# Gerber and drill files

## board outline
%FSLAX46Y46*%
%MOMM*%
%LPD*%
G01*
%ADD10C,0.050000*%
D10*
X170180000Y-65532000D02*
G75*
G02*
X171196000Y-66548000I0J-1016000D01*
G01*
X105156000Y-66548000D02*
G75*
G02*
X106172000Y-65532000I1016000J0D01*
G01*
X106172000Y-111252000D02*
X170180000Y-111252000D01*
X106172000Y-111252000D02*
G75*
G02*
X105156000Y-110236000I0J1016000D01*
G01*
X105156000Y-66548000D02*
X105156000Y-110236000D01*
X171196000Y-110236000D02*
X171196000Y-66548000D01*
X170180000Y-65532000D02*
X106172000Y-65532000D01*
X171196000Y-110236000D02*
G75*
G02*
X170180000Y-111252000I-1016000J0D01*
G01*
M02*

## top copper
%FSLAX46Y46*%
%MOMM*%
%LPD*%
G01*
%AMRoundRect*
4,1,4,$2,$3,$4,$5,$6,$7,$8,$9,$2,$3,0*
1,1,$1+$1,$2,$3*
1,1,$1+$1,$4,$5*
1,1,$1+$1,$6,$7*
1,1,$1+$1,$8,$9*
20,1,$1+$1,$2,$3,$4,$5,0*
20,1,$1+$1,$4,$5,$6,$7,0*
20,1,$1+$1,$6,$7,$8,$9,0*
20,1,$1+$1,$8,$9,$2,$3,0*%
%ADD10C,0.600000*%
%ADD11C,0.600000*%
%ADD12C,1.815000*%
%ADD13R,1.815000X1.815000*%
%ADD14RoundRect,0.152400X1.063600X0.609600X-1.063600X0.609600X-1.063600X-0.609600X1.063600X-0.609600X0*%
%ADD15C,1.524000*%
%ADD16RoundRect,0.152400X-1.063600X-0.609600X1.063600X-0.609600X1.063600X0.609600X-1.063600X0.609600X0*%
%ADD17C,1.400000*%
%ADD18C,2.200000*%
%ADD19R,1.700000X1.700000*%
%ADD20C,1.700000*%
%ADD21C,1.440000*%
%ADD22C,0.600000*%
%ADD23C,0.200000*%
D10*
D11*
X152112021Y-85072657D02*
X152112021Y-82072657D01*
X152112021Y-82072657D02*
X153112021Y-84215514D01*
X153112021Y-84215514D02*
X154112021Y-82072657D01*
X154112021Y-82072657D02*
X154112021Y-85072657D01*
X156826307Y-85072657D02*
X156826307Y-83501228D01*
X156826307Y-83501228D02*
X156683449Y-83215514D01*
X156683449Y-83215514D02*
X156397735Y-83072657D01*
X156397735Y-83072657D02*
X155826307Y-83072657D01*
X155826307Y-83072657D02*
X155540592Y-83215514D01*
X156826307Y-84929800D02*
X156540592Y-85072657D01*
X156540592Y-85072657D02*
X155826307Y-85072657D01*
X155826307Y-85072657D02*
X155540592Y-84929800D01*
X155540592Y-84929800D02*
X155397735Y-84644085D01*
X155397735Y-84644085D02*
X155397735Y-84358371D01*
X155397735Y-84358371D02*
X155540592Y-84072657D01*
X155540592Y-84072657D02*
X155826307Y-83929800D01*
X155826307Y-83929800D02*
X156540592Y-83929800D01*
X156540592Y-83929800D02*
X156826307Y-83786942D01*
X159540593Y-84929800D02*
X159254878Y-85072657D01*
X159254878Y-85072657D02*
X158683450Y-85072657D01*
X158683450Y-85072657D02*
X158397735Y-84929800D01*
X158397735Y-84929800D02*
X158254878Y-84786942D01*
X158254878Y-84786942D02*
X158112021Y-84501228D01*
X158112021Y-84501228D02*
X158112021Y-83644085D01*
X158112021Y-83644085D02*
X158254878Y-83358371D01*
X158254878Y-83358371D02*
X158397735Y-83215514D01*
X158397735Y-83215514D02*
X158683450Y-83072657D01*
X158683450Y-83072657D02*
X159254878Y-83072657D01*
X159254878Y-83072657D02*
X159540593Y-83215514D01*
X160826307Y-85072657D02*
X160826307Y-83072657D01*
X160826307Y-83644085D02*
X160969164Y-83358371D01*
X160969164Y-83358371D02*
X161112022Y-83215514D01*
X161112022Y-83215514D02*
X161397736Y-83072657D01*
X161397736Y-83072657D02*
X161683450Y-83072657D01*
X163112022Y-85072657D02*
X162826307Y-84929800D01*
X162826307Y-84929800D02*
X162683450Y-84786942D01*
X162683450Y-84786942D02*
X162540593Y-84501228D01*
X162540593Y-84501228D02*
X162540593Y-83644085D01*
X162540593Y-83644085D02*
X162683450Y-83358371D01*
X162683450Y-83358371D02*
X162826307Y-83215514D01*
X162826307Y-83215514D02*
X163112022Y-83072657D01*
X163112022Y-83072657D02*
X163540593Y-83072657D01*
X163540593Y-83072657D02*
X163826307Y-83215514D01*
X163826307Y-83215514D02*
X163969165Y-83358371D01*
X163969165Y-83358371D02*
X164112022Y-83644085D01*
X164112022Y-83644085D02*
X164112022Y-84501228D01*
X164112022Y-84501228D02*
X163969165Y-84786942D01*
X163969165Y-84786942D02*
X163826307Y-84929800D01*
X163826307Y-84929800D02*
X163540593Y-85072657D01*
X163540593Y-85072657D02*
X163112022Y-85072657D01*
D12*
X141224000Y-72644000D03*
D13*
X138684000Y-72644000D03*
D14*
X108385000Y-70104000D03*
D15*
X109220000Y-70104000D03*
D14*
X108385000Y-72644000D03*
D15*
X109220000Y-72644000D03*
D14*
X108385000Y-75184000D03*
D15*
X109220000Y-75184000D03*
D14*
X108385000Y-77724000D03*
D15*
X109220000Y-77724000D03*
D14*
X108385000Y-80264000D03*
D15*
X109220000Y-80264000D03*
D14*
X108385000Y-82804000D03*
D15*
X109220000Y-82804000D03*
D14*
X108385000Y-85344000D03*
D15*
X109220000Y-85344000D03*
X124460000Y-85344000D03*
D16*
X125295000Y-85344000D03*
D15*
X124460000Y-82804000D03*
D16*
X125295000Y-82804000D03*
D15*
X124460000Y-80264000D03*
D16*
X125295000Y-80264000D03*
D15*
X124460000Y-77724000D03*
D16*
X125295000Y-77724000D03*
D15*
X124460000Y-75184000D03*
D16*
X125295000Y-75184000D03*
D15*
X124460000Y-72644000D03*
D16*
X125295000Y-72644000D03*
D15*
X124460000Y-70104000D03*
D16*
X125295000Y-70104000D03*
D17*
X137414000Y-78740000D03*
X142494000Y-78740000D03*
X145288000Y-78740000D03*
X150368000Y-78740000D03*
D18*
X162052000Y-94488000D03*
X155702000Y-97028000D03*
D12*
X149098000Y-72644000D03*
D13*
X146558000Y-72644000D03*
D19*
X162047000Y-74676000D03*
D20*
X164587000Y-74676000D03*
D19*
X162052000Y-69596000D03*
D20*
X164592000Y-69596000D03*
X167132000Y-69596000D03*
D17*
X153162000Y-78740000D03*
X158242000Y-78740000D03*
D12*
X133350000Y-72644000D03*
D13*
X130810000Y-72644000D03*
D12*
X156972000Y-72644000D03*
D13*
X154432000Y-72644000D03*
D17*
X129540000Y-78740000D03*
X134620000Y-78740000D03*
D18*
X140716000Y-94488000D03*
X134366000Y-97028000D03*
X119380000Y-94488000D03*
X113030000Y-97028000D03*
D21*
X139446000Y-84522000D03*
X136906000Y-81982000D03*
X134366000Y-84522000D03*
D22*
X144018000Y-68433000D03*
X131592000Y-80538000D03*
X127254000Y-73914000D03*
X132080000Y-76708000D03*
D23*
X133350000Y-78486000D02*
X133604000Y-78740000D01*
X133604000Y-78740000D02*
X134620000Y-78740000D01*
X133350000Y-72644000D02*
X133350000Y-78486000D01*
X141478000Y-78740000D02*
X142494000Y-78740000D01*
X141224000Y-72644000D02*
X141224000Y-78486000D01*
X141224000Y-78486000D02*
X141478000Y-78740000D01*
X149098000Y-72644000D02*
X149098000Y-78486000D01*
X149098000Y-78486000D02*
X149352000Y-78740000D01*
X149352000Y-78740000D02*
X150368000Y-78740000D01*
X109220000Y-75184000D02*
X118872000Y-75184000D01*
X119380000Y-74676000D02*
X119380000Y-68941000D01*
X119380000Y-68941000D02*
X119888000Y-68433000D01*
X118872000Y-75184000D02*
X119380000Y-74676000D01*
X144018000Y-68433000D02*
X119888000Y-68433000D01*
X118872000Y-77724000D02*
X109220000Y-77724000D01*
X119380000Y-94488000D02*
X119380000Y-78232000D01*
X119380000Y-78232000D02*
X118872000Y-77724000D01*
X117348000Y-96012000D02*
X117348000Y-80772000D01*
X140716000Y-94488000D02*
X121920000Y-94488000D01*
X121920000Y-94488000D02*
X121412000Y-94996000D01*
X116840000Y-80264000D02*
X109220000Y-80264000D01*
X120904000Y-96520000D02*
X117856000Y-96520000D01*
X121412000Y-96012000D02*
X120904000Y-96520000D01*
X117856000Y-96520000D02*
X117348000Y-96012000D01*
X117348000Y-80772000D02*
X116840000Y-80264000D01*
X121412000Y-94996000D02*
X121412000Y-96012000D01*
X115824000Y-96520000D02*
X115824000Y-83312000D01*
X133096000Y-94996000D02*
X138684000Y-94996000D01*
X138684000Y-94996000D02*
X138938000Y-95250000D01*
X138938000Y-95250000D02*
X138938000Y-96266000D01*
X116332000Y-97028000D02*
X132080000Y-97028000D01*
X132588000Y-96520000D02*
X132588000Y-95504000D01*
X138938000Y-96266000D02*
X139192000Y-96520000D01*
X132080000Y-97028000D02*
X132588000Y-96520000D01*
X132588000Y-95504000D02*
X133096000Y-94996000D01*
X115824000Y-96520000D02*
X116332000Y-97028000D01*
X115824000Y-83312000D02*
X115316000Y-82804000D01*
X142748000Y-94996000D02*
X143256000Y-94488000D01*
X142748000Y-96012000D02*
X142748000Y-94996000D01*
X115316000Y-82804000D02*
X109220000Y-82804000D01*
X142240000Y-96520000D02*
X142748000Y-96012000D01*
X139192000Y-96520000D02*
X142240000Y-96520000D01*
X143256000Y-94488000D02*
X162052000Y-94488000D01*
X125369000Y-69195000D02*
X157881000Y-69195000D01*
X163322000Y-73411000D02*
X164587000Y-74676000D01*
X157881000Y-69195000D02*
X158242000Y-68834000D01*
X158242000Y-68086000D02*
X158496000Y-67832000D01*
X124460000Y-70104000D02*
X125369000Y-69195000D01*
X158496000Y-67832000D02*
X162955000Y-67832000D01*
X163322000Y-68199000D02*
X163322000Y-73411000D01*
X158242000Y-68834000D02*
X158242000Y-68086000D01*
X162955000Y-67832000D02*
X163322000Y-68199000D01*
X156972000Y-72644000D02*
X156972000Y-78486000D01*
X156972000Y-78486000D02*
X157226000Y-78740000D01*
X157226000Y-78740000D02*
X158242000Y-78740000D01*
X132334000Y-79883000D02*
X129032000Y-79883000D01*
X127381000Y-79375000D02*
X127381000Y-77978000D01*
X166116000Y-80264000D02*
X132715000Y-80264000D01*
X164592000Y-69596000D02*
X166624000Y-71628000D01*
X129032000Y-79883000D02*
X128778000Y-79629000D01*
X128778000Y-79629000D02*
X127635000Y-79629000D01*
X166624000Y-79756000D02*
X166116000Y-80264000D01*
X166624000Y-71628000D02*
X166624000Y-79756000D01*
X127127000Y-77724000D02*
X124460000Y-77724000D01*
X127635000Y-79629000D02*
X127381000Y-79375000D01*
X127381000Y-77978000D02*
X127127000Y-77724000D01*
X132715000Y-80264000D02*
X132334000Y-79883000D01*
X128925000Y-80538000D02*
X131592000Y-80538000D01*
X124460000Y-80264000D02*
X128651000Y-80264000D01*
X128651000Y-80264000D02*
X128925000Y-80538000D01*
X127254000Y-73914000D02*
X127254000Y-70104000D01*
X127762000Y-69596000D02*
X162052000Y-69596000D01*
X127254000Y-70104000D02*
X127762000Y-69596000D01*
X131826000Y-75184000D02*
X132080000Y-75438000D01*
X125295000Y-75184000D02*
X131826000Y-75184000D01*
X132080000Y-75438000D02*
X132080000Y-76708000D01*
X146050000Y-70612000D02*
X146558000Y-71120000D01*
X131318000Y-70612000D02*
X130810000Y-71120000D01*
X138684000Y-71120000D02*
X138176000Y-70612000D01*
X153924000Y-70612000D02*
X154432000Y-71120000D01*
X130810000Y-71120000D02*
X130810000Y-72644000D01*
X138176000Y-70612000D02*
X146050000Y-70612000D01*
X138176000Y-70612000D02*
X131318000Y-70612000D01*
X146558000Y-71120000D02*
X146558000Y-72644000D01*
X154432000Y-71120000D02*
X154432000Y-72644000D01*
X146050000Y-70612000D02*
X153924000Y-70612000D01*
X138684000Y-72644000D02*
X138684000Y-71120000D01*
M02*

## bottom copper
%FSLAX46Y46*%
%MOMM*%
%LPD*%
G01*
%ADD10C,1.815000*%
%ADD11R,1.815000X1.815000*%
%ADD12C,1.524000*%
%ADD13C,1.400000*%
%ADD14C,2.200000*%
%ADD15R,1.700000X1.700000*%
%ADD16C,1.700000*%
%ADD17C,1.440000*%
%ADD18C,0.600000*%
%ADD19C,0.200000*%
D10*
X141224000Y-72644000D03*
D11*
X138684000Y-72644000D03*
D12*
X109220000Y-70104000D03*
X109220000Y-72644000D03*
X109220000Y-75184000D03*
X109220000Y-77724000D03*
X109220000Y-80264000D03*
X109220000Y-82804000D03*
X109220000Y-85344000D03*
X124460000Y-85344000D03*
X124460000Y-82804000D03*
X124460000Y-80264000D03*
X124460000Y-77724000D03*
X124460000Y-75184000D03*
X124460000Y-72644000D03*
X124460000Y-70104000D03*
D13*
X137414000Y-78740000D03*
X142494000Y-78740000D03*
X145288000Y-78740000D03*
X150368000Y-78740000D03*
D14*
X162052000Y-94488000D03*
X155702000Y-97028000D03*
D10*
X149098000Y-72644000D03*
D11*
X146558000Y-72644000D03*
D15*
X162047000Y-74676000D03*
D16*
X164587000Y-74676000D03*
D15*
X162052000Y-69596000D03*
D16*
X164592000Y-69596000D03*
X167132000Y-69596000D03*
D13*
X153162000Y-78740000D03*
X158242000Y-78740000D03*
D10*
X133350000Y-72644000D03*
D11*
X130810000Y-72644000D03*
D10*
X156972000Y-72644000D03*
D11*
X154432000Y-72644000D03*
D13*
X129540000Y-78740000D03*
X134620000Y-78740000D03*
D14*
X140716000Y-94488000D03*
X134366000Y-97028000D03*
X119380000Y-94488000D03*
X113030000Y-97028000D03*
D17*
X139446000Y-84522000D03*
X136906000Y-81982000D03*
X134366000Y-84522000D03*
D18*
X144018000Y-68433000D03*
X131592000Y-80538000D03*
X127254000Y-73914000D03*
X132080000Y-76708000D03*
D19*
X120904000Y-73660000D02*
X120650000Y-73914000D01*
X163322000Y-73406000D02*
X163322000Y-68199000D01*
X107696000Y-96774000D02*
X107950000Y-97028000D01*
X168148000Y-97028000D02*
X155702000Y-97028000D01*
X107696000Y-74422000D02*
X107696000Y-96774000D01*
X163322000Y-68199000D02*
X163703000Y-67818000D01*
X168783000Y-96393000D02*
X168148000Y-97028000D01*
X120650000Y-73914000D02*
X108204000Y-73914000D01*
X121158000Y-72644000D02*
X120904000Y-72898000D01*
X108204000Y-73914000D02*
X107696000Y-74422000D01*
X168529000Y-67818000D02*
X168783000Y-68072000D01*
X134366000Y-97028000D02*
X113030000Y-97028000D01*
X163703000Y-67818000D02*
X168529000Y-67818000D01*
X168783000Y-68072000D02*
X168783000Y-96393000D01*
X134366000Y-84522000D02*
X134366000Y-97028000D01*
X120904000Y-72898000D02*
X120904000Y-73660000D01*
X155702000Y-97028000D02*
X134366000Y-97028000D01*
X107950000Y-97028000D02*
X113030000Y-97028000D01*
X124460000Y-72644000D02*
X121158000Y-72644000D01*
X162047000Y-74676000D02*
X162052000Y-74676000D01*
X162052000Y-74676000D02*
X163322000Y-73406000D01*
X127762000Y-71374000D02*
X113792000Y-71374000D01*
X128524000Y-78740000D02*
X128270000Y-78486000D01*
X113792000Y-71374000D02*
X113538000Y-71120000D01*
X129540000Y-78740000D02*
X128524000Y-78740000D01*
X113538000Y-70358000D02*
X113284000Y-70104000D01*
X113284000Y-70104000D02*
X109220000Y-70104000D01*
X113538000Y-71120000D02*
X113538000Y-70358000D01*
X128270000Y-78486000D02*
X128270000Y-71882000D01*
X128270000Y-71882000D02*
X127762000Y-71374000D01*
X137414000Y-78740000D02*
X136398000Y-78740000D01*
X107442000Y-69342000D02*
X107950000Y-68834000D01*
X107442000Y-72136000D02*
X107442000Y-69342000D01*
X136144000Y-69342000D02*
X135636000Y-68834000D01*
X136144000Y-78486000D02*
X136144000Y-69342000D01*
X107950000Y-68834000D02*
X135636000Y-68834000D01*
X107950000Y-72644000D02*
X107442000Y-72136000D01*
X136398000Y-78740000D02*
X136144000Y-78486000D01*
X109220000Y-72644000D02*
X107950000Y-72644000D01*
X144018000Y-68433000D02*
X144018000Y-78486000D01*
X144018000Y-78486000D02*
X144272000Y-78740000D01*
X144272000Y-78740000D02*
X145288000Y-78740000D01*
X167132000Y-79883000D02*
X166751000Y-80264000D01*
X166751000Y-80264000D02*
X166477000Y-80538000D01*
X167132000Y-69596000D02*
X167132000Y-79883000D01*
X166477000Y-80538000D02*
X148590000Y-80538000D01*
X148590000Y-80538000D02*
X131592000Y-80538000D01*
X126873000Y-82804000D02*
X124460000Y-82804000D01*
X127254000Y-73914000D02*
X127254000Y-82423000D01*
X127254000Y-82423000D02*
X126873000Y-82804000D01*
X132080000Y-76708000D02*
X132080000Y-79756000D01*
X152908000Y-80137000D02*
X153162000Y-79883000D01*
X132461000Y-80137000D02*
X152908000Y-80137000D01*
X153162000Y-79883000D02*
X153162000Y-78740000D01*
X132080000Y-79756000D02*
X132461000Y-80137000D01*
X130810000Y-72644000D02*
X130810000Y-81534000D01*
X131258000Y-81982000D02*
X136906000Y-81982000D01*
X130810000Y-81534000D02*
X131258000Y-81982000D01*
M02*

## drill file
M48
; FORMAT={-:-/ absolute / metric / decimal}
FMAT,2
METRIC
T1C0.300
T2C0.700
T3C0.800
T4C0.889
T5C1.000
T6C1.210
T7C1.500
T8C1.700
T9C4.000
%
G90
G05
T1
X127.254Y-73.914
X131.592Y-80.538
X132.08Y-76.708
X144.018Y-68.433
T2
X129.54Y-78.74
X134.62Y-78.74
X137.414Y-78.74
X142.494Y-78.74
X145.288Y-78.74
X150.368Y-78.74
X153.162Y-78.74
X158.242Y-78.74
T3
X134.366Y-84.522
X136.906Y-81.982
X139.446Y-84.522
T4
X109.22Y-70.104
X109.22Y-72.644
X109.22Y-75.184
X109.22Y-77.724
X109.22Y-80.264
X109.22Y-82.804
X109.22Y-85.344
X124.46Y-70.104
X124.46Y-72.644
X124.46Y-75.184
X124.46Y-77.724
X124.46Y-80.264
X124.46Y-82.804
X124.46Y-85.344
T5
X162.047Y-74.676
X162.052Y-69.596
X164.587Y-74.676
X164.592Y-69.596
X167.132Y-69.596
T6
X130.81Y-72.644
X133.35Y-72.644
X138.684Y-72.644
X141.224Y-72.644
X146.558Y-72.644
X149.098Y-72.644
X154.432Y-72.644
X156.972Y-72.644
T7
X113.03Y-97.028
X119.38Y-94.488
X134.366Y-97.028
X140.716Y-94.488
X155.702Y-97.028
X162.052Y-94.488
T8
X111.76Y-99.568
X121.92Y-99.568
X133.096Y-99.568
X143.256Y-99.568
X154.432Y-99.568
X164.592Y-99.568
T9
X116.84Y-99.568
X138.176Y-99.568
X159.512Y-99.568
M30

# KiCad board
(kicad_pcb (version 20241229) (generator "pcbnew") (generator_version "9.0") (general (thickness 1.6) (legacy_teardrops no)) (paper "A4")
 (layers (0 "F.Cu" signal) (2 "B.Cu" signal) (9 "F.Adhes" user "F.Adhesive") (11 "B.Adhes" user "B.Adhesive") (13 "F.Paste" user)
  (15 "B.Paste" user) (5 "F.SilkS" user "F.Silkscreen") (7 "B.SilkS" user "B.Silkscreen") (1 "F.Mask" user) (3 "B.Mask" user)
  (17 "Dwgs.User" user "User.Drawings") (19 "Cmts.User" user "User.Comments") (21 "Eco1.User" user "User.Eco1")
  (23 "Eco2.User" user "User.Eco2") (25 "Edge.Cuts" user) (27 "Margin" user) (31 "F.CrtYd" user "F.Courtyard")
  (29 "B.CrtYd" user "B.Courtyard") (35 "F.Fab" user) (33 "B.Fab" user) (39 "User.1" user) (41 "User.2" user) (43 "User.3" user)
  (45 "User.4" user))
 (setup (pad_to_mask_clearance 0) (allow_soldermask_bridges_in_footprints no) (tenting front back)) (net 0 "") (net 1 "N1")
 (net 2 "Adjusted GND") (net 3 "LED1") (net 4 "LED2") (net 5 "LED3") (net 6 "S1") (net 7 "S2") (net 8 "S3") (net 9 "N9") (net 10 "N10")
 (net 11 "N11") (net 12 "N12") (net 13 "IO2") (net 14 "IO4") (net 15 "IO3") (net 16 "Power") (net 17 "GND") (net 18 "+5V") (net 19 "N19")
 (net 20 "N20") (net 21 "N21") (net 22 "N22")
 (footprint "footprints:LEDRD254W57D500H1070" (layer "F.Cu") (at 139.954 72.644)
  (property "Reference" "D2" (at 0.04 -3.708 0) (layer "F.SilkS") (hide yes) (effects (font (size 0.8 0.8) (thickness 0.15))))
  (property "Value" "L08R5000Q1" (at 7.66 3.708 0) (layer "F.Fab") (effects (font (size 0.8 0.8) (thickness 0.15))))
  (pad "A" thru_hole circle (at 1.27 0) (size 1.815 1.815) (drill 1.21) (layers "*.Cu" "*.Mask") (remove_unused_layers no) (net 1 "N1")
   (solder_mask_margin 0.102))
  (pad "C" thru_hole rect (at -1.27 0) (size 1.815 1.815) (drill 1.21) (layers "*.Cu" "*.Mask") (remove_unused_layers no)
   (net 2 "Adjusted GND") (solder_mask_margin 0.102)))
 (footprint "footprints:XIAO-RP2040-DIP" (layer "F.Cu") (at 116.84 77.724)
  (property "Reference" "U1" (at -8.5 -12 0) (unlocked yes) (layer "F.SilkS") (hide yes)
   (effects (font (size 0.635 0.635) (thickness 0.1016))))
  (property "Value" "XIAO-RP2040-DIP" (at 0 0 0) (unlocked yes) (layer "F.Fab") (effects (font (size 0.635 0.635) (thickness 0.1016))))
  (pad "1" smd roundrect (at -8.455 -7.62 180) (size 2.432 1.524) (layers "F.Cu" "F.Mask") (roundrect_rratio 0.1) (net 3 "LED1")
   (thermal_bridge_angle 45))
  (pad "1" thru_hole circle (at -7.62 -7.62 180) (size 1.524 1.524) (drill 0.889) (layers "*.Cu" "*.Mask") (remove_unused_layers no)
   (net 3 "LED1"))
  (pad "2" smd roundrect (at -8.455 -5.08 180) (size 2.432 1.524) (layers "F.Cu" "F.Mask") (roundrect_rratio 0.1) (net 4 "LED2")
   (thermal_bridge_angle 45))
  (pad "2" thru_hole circle (at -7.62 -5.08 180) (size 1.524 1.524) (drill 0.889) (layers "*.Cu" "*.Mask") (remove_unused_layers no)
   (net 4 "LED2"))
  (pad "3" smd roundrect (at -8.455 -2.54 180) (size 2.432 1.524) (layers "F.Cu" "F.Mask") (roundrect_rratio 0.1) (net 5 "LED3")
   (thermal_bridge_angle 45))
  (pad "3" thru_hole circle (at -7.62 -2.54 180) (size 1.524 1.524) (drill 0.889) (layers "*.Cu" "*.Mask") (remove_unused_layers no)
   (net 5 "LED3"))
  (pad "4" smd roundrect (at -8.455 0 180) (size 2.432 1.524) (layers "F.Cu" "F.Mask") (roundrect_rratio 0.1) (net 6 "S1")
   (thermal_bridge_angle 45))
  (pad "4" thru_hole circle (at -7.62 0 180) (size 1.524 1.524) (drill 0.889) (layers "*.Cu" "*.Mask") (remove_unused_layers no)
   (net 6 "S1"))
  (pad "5" smd roundrect (at -8.455 2.54 180) (size 2.432 1.524) (layers "F.Cu" "F.Mask") (roundrect_rratio 0.1) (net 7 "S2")
   (thermal_bridge_angle 45))
  (pad "5" thru_hole circle (at -7.62 2.54 180) (size 1.524 1.524) (drill 0.889) (layers "*.Cu" "*.Mask") (remove_unused_layers no)
   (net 7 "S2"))
  (pad "6" smd roundrect (at -8.455 5.08 180) (size 2.432 1.524) (layers "F.Cu" "F.Mask") (roundrect_rratio 0.1) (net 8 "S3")
   (thermal_bridge_angle 45))
  (pad "6" thru_hole circle (at -7.62 5.08 180) (size 1.524 1.524) (drill 0.889) (layers "*.Cu" "*.Mask") (remove_unused_layers no)
   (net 8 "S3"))
  (pad "7" smd roundrect (at -8.455 7.62 180) (size 2.432 1.524) (layers "F.Cu" "F.Mask") (roundrect_rratio 0.1) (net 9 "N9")
   (thermal_bridge_angle 45))
  (pad "7" thru_hole circle (at -7.62 7.62 180) (size 1.524 1.524) (drill 0.889) (layers "*.Cu" "*.Mask") (remove_unused_layers no)
   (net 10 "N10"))
  (pad "8" thru_hole circle (at 7.62 7.62) (size 1.524 1.524) (drill 0.889) (layers "*.Cu" "*.Mask") (remove_unused_layers no)
   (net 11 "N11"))
  (pad "8" smd roundrect (at 8.455 7.62) (size 2.432 1.524) (layers "F.Cu" "F.Mask") (roundrect_rratio 0.1) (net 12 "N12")
   (thermal_bridge_angle 45))
  (pad "9" thru_hole circle (at 7.62 5.08) (size 1.524 1.524) (drill 0.889) (layers "*.Cu" "*.Mask") (remove_unused_layers no)
   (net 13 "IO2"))
  (pad "9" smd roundrect (at 8.455 5.08) (size 2.432 1.524) (layers "F.Cu" "F.Mask") (roundrect_rratio 0.1) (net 13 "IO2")
   (thermal_bridge_angle 45))
  (pad "10" thru_hole circle (at 7.62 2.54) (size 1.524 1.524) (drill 0.889) (layers "*.Cu" "*.Mask") (remove_unused_layers no)
   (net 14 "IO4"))
  (pad "10" smd roundrect (at 8.455 2.54) (size 2.432 1.524) (layers "F.Cu" "F.Mask") (roundrect_rratio 0.1) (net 14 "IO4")
   (thermal_bridge_angle 45))
  (pad "11" thru_hole circle (at 7.62 0) (size 1.524 1.524) (drill 0.889) (layers "*.Cu" "*.Mask") (remove_unused_layers no) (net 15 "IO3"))
  (pad "11" smd roundrect (at 8.455 0) (size 2.432 1.524) (layers "F.Cu" "F.Mask") (roundrect_rratio 0.1) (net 15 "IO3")
   (thermal_bridge_angle 45))
  (pad "12" thru_hole circle (at 7.62 -2.54) (size 1.524 1.524) (drill 0.889) (layers "*.Cu" "*.Mask") (remove_unused_layers no)
   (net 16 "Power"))
  (pad "12" smd roundrect (at 8.455 -2.54) (size 2.432 1.524) (layers "F.Cu" "F.Mask") (roundrect_rratio 0.1) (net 16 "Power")
   (thermal_bridge_angle 45))
  (pad "13" thru_hole circle (at 7.62 -5.08) (size 1.524 1.524) (drill 0.889) (layers "*.Cu" "*.Mask") (remove_unused_layers no)
   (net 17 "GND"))
  (pad "13" smd roundrect (at 8.455 -5.08) (size 2.432 1.524) (layers "F.Cu" "F.Mask") (roundrect_rratio 0.1) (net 17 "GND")
   (thermal_bridge_angle 45))
  (pad "14" thru_hole circle (at 7.62 -7.62) (size 1.524 1.524) (drill 0.889) (layers "*.Cu" "*.Mask") (remove_unused_layers no)
   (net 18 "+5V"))
  (pad "14" smd roundrect (at 8.455 -7.62) (size 2.432 1.524) (layers "F.Cu" "F.Mask") (roundrect_rratio 0.1) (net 18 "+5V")
   (thermal_bridge_angle 45)))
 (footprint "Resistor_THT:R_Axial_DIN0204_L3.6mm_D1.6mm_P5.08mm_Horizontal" (layer "F.Cu") (at 137.414 78.74)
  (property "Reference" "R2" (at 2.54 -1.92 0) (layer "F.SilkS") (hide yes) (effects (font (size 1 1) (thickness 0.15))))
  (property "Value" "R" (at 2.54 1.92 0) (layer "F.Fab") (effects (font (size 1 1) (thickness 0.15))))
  (pad "1" thru_hole circle (at 0 0) (size 1.4 1.4) (drill 0.7) (layers "*.Cu" "*.Mask") (remove_unused_layers no) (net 4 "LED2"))
  (pad "2" thru_hole circle (at 5.08 0) (size 1.4 1.4) (drill 0.7) (layers "*.Cu" "*.Mask") (remove_unused_layers no) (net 1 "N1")))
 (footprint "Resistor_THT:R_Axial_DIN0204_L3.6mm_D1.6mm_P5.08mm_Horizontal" (layer "F.Cu") (at 145.288 78.74)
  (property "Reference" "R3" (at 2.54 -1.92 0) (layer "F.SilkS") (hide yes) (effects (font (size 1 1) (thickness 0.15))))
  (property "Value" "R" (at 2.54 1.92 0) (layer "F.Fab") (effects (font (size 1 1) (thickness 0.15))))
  (pad "1" thru_hole circle (at 0 0) (size 1.4 1.4) (drill 0.7) (layers "*.Cu" "*.Mask") (remove_unused_layers no) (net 5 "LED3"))
  (pad "2" thru_hole circle (at 5.08 0) (size 1.4 1.4) (drill 0.7) (layers "*.Cu" "*.Mask") (remove_unused_layers no) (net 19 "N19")))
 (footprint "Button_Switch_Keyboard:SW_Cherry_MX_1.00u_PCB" (layer "F.Cu") (at 162.052 94.488)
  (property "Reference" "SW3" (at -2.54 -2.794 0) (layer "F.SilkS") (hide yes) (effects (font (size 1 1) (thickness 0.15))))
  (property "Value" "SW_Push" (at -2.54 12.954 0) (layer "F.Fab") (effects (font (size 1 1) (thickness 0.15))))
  (pad "" np_thru_hole circle (at -7.62 5.08) (size 1.7 1.7) (drill 1.7) (layers "*.Cu" "*.Mask"))
  (pad "" np_thru_hole circle (at -2.54 5.08) (size 4 4) (drill 4) (layers "*.Cu" "*.Mask"))
  (pad "" np_thru_hole circle (at 2.54 5.08) (size 1.7 1.7) (drill 1.7) (layers "*.Cu" "*.Mask"))
  (pad "1" thru_hole circle (at 0 0) (size 2.2 2.2) (drill 1.5) (layers "*.Cu" "*.Mask") (remove_unused_layers no) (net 8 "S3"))
  (pad "2" thru_hole circle (at -6.35 2.54) (size 2.2 2.2) (drill 1.5) (layers "*.Cu" "*.Mask") (remove_unused_layers no) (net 17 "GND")))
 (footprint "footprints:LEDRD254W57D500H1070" (layer "F.Cu") (at 147.828 72.644)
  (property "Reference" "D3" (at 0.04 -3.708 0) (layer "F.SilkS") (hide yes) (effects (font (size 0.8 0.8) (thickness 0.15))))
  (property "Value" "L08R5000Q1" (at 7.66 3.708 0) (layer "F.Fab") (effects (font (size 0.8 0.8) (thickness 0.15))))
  (pad "A" thru_hole circle (at 1.27 0) (size 1.815 1.815) (drill 1.21) (layers "*.Cu" "*.Mask") (remove_unused_layers no) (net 19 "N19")
   (solder_mask_margin 0.102))
  (pad "C" thru_hole rect (at -1.27 0) (size 1.815 1.815) (drill 1.21) (layers "*.Cu" "*.Mask") (remove_unused_layers no)
   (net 2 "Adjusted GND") (solder_mask_margin 0.102)))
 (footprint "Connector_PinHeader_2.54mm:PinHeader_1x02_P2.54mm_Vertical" (layer "F.Cu") (at 162.047 74.676 90)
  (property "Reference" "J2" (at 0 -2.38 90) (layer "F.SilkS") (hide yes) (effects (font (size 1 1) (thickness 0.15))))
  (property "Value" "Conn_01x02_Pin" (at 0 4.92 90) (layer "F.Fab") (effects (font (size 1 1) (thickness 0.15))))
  (pad "1" thru_hole rect (at 0 0 90) (size 1.7 1.7) (drill 1) (layers "*.Cu" "*.Mask") (remove_unused_layers no) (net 17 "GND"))
  (pad "2" thru_hole circle (at 0 2.54 90) (size 1.7 1.7) (drill 1) (layers "*.Cu" "*.Mask") (remove_unused_layers no) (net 18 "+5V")))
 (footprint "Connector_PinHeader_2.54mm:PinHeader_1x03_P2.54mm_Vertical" (layer "F.Cu") (at 162.052 69.596 90)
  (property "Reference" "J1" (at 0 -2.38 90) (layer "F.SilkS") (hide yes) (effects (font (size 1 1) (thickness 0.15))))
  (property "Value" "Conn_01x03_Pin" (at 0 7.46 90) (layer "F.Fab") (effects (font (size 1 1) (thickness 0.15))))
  (pad "1" thru_hole rect (at 0 0 90) (size 1.7 1.7) (drill 1) (layers "*.Cu" "*.Mask") (remove_unused_layers no) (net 13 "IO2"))
  (pad "2" thru_hole circle (at 0 2.54 90) (size 1.7 1.7) (drill 1) (layers "*.Cu" "*.Mask") (remove_unused_layers no) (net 15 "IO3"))
  (pad "3" thru_hole circle (at 0 5.08 90) (size 1.7 1.7) (drill 1) (layers "*.Cu" "*.Mask") (remove_unused_layers no) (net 14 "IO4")))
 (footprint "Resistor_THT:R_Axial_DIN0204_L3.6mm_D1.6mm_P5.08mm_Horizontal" (layer "F.Cu") (at 153.162 78.74)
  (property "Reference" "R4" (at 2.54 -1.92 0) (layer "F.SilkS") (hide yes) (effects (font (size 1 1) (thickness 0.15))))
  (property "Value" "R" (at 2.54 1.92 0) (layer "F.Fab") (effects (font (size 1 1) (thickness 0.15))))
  (pad "1" thru_hole circle (at 0 0) (size 1.4 1.4) (drill 0.7) (layers "*.Cu" "*.Mask") (remove_unused_layers no) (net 16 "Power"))
  (pad "2" thru_hole circle (at 5.08 0) (size 1.4 1.4) (drill 0.7) (layers "*.Cu" "*.Mask") (remove_unused_layers no) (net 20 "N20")))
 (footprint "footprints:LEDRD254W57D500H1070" (layer "F.Cu") (at 132.08 72.644)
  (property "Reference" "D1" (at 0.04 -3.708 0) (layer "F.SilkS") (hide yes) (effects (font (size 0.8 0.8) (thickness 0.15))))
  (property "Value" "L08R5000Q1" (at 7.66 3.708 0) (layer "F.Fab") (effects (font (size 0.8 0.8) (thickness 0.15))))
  (pad "A" thru_hole circle (at 1.27 0) (size 1.815 1.815) (drill 1.21) (layers "*.Cu" "*.Mask") (remove_unused_layers no) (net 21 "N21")
   (solder_mask_margin 0.102))
  (pad "C" thru_hole rect (at -1.27 0) (size 1.815 1.815) (drill 1.21) (layers "*.Cu" "*.Mask") (remove_unused_layers no)
   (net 2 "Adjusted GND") (solder_mask_margin 0.102)))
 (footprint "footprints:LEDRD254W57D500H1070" (layer "F.Cu") (at 155.702 72.644)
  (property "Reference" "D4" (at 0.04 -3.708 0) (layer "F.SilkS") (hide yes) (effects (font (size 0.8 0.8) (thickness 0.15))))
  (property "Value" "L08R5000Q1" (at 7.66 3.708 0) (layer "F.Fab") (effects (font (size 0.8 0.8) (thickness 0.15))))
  (pad "A" thru_hole circle (at 1.27 0) (size 1.815 1.815) (drill 1.21) (layers "*.Cu" "*.Mask") (remove_unused_layers no) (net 20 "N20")
   (solder_mask_margin 0.102))
  (pad "C" thru_hole rect (at -1.27 0) (size 1.815 1.815) (drill 1.21) (layers "*.Cu" "*.Mask") (remove_unused_layers no)
   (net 2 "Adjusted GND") (solder_mask_margin 0.102)))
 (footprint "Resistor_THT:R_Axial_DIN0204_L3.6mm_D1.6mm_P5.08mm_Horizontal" (layer "F.Cu") (at 129.54 78.74)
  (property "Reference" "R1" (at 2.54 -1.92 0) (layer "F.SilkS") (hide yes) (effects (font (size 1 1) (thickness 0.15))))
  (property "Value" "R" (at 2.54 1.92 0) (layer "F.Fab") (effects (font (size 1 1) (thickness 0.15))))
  (pad "1" thru_hole circle (at 0 0) (size 1.4 1.4) (drill 0.7) (layers "*.Cu" "*.Mask") (remove_unused_layers no) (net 3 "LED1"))
  (pad "2" thru_hole circle (at 5.08 0) (size 1.4 1.4) (drill 0.7) (layers "*.Cu" "*.Mask") (remove_unused_layers no) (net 21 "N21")))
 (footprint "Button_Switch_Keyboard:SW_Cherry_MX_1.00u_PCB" (layer "F.Cu") (at 140.716 94.488)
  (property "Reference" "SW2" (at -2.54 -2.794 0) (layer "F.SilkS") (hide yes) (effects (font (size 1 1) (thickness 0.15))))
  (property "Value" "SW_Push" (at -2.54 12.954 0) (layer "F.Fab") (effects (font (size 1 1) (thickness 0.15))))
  (pad "" np_thru_hole circle (at -7.62 5.08) (size 1.7 1.7) (drill 1.7) (layers "*.Cu" "*.Mask"))
  (pad "" np_thru_hole circle (at -2.54 5.08) (size 4 4) (drill 4) (layers "*.Cu" "*.Mask"))
  (pad "" np_thru_hole circle (at 2.54 5.08) (size 1.7 1.7) (drill 1.7) (layers "*.Cu" "*.Mask"))
  (pad "1" thru_hole circle (at 0 0) (size 2.2 2.2) (drill 1.5) (layers "*.Cu" "*.Mask") (remove_unused_layers no) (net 7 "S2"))
  (pad "2" thru_hole circle (at -6.35 2.54) (size 2.2 2.2) (drill 1.5) (layers "*.Cu" "*.Mask") (remove_unused_layers no) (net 17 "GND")))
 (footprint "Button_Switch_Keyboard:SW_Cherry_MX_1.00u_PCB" (layer "F.Cu") (at 119.38 94.488)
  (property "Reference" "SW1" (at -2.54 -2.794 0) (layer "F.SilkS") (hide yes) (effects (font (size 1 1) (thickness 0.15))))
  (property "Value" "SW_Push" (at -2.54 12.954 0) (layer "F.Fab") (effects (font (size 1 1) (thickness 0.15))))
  (pad "" np_thru_hole circle (at -7.62 5.08) (size 1.7 1.7) (drill 1.7) (layers "*.Cu" "*.Mask"))
  (pad "" np_thru_hole circle (at -2.54 5.08) (size 4 4) (drill 4) (layers "*.Cu" "*.Mask"))
  (pad "" np_thru_hole circle (at 2.54 5.08) (size 1.7 1.7) (drill 1.7) (layers "*.Cu" "*.Mask"))
  (pad "1" thru_hole circle (at 0 0) (size 2.2 2.2) (drill 1.5) (layers "*.Cu" "*.Mask") (remove_unused_layers no) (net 6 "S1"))
  (pad "2" thru_hole circle (at -6.35 2.54) (size 2.2 2.2) (drill 1.5) (layers "*.Cu" "*.Mask") (remove_unused_layers no) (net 17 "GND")))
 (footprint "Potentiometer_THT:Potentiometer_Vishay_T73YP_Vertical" (layer "F.Cu") (at 139.446 84.522 90)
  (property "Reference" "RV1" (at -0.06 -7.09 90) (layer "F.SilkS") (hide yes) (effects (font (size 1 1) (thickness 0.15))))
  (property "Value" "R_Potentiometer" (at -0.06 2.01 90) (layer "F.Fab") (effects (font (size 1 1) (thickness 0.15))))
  (pad "1" thru_hole circle (at 0 0 90) (size 1.44 1.44) (drill 0.8) (layers "*.Cu" "*.Mask") (remove_unused_layers no) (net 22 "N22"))
  (pad "2" thru_hole circle (at 2.54 -2.54 90) (size 1.44 1.44) (drill 0.8) (layers "*.Cu" "*.Mask") (remove_unused_layers no)
   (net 2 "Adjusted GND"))
  (pad "3" thru_hole circle (at 0 -5.08 90) (size 1.44 1.44) (drill 0.8) (layers "*.Cu" "*.Mask") (remove_unused_layers no) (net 17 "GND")))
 (gr_arc (start 170.18 65.532) (mid 170.89842 65.82958) (end 171.196 66.548) (stroke (width 0.05) (type default)) (layer "Edge.Cuts"))
 (gr_arc (start 105.156 66.548) (mid 105.45358 65.82958) (end 106.172 65.532) (stroke (width 0.05) (type default)) (layer "Edge.Cuts"))
 (gr_line (start 106.172 111.252) (end 170.18 111.252) (stroke (width 0.05) (type default)) (layer "Edge.Cuts"))
 (gr_arc (start 106.172 111.252) (mid 105.45358 110.95442) (end 105.156 110.236) (stroke (width 0.05) (type default)) (layer "Edge.Cuts"))
 (gr_line (start 105.156 66.548) (end 105.156 110.236) (stroke (width 0.05) (type default)) (layer "Edge.Cuts"))
 (gr_line (start 171.196 110.236) (end 171.196 66.548) (stroke (width 0.05) (type default)) (layer "Edge.Cuts"))
 (gr_line (start 170.18 65.532) (end 106.172 65.532) (stroke (width 0.05) (type default)) (layer "Edge.Cuts"))
 (gr_arc (start 171.196 110.236) (mid 170.89842 110.95442) (end 170.18 111.252) (stroke (width 0.05) (type default)) (layer "Edge.Cuts"))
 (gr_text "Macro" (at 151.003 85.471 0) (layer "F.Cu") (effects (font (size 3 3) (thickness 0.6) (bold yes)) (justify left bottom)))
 (segment (start 120.904 73.66) (end 120.65 73.914) (width 0.2) (layer "B.Cu") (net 17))
 (segment (start 163.322 73.406) (end 163.322 68.199) (width 0.2) (layer "B.Cu") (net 17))
 (segment (start 107.696 96.774) (end 107.95 97.028) (width 0.2) (layer "B.Cu") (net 17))
 (segment (start 168.148 97.028) (end 155.702 97.028) (width 0.2) (layer "B.Cu") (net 17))
 (segment (start 107.696 74.422) (end 107.696 96.774) (width 0.2) (layer "B.Cu") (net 17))
 (segment (start 163.322 68.199) (end 163.703 67.818) (width 0.2) (layer "B.Cu") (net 17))
 (segment (start 168.783 96.393) (end 168.148 97.028) (width 0.2) (layer "B.Cu") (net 17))
 (segment (start 120.65 73.914) (end 108.204 73.914) (width 0.2) (layer "B.Cu") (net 17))
 (segment (start 121.158 72.644) (end 120.904 72.898) (width 0.2) (layer "B.Cu") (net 17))
 (segment (start 108.204 73.914) (end 107.696 74.422) (width 0.2) (layer "B.Cu") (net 17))
 (segment (start 168.529 67.818) (end 168.783 68.072) (width 0.2) (layer "B.Cu") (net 17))
 (segment (start 134.366 97.028) (end 113.03 97.028) (width 0.2) (layer "B.Cu") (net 17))
 (segment (start 163.703 67.818) (end 168.529 67.818) (width 0.2) (layer "B.Cu") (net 17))
 (segment (start 168.783 68.072) (end 168.783 96.393) (width 0.2) (layer "B.Cu") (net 17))
 (segment (start 134.366 84.522) (end 134.366 97.028) (width 0.2) (layer "B.Cu") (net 17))
 (segment (start 120.904 72.898) (end 120.904 73.66) (width 0.2) (layer "B.Cu") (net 17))
 (segment (start 155.702 97.028) (end 134.366 97.028) (width 0.2) (layer "B.Cu") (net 17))
 (segment (start 107.95 97.028) (end 113.03 97.028) (width 0.2) (layer "B.Cu") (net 17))
 (segment (start 124.46 72.644) (end 121.158 72.644) (width 0.2) (layer "B.Cu") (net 17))
 (segment (start 162.047 74.676) (end 162.052 74.676) (width 0.2) (layer "B.Cu") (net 17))
 (segment (start 162.052 74.676) (end 163.322 73.406) (width 0.2) (layer "B.Cu") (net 17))
 (segment (start 133.35 78.486) (end 133.604 78.74) (width 0.2) (layer "F.Cu") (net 21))
 (segment (start 133.604 78.74) (end 134.62 78.74) (width 0.2) (layer "F.Cu") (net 21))
 (segment (start 133.35 72.644) (end 133.35 78.486) (width 0.2) (layer "F.Cu") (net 21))
 (segment (start 141.478 78.74) (end 142.494 78.74) (width 0.2) (layer "F.Cu") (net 1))
 (segment (start 141.224 72.644) (end 141.224 78.486) (width 0.2) (layer "F.Cu") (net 1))
 (segment (start 141.224 78.486) (end 141.478 78.74) (width 0.2) (layer "F.Cu") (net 1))
 (segment (start 149.098 72.644) (end 149.098 78.486) (width 0.2) (layer "F.Cu") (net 19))
 (segment (start 149.098 78.486) (end 149.352 78.74) (width 0.2) (layer "F.Cu") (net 19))
 (segment (start 149.352 78.74) (end 150.368 78.74) (width 0.2) (layer "F.Cu") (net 19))
 (segment (start 127.762 71.374) (end 113.792 71.374) (width 0.2) (layer "B.Cu") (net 3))
 (segment (start 128.524 78.74) (end 128.27 78.486) (width 0.2) (layer "B.Cu") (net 3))
 (segment (start 113.792 71.374) (end 113.538 71.12) (width 0.2) (layer "B.Cu") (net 3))
 (segment (start 129.54 78.74) (end 128.524 78.74) (width 0.2) (layer "B.Cu") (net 3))
 (segment (start 113.538 70.358) (end 113.284 70.104) (width 0.2) (layer "B.Cu") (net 3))
 (segment (start 113.284 70.104) (end 109.22 70.104) (width 0.2) (layer "B.Cu") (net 3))
 (segment (start 113.538 71.12) (end 113.538 70.358) (width 0.2) (layer "B.Cu") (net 3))
 (segment (start 128.27 78.486) (end 128.27 71.882) (width 0.2) (layer "B.Cu") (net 3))
 (segment (start 128.27 71.882) (end 127.762 71.374) (width 0.2) (layer "B.Cu") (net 3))
 (segment (start 137.414 78.74) (end 136.398 78.74) (width 0.2) (layer "B.Cu") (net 4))
 (segment (start 107.442 69.342) (end 107.95 68.834) (width 0.2) (layer "B.Cu") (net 4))
 (segment (start 107.442 72.136) (end 107.442 69.342) (width 0.2) (layer "B.Cu") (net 4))
 (segment (start 136.144 69.342) (end 135.636 68.834) (width 0.2) (layer "B.Cu") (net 4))
 (segment (start 136.144 78.486) (end 136.144 69.342) (width 0.2) (layer "B.Cu") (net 4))
 (segment (start 107.95 68.834) (end 135.636 68.834) (width 0.2) (layer "B.Cu") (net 4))
 (segment (start 107.95 72.644) (end 107.442 72.136) (width 0.2) (layer "B.Cu") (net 4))
 (segment (start 136.398 78.74) (end 136.144 78.486) (width 0.2) (layer "B.Cu") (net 4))
 (segment (start 109.22 72.644) (end 107.95 72.644) (width 0.2) (layer "B.Cu") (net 4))
 (segment (start 109.22 75.184) (end 118.872 75.184) (width 0.2) (layer "F.Cu") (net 5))
 (segment (start 119.38 74.676) (end 119.38 68.941) (width 0.2) (layer "F.Cu") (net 5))
 (segment (start 119.38 68.941) (end 119.888 68.433) (width 0.2) (layer "F.Cu") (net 5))
 (segment (start 118.872 75.184) (end 119.38 74.676) (width 0.2) (layer "F.Cu") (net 5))
 (segment (start 144.018 68.433) (end 119.888 68.433) (width 0.2) (layer "F.Cu") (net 5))
 (via (at 144.018 68.433) (size 0.6) (drill 0.3) (layers "F.Cu" "B.Cu") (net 5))
 (segment (start 144.018 68.433) (end 144.018 78.486) (width 0.2) (layer "B.Cu") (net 5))
 (segment (start 144.018 78.486) (end 144.272 78.74) (width 0.2) (layer "B.Cu") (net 5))
 (segment (start 144.272 78.74) (end 145.288 78.74) (width 0.2) (layer "B.Cu") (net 5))
 (segment (start 118.872 77.724) (end 109.22 77.724) (width 0.2) (layer "F.Cu") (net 6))
 (segment (start 119.38 94.488) (end 119.38 78.232) (width 0.2) (layer "F.Cu") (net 6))
 (segment (start 119.38 78.232) (end 118.872 77.724) (width 0.2) (layer "F.Cu") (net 6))
 (segment (start 117.348 96.012) (end 117.348 80.772) (width 0.2) (layer "F.Cu") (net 7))
 (segment (start 140.716 94.488) (end 121.92 94.488) (width 0.2) (layer "F.Cu") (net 7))
 (segment (start 121.92 94.488) (end 121.412 94.996) (width 0.2) (layer "F.Cu") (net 7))
 (segment (start 116.84 80.264) (end 109.22 80.264) (width 0.2) (layer "F.Cu") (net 7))
 (segment (start 120.904 96.52) (end 117.856 96.52) (width 0.2) (layer "F.Cu") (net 7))
 (segment (start 121.412 96.012) (end 120.904 96.52) (width 0.2) (layer "F.Cu") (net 7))
 (segment (start 117.856 96.52) (end 117.348 96.012) (width 0.2) (layer "F.Cu") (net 7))
 (segment (start 117.348 80.772) (end 116.84 80.264) (width 0.2) (layer "F.Cu") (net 7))
 (segment (start 121.412 94.996) (end 121.412 96.012) (width 0.2) (layer "F.Cu") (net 7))
 (segment (start 115.824 96.52) (end 115.824 83.312) (width 0.2) (layer "F.Cu") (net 8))
 (segment (start 133.096 94.996) (end 138.684 94.996) (width 0.2) (layer "F.Cu") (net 8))
 (segment (start 138.684 94.996) (end 138.938 95.25) (width 0.2) (layer "F.Cu") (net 8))
 (segment (start 138.938 95.25) (end 138.938 96.266) (width 0.2) (layer "F.Cu") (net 8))
 (segment (start 116.332 97.028) (end 132.08 97.028) (width 0.2) (layer "F.Cu") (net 8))
 (segment (start 132.588 96.52) (end 132.588 95.504) (width 0.2) (layer "F.Cu") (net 8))
 (segment (start 138.938 96.266) (end 139.192 96.52) (width 0.2) (layer "F.Cu") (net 8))
 (segment (start 132.08 97.028) (end 132.588 96.52) (width 0.2) (layer "F.Cu") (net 8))
 (segment (start 132.588 95.504) (end 133.096 94.996) (width 0.2) (layer "F.Cu") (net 8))
 (segment (start 115.824 96.52) (end 116.332 97.028) (width 0.2) (layer "F.Cu") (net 8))
 (segment (start 115.824 83.312) (end 115.316 82.804) (width 0.2) (layer "F.Cu") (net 8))
 (segment (start 142.748 94.996) (end 143.256 94.488) (width 0.2) (layer "F.Cu") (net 8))
 (segment (start 142.748 96.012) (end 142.748 94.996) (width 0.2) (layer "F.Cu") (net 8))
 (segment (start 115.316 82.804) (end 109.22 82.804) (width 0.2) (layer "F.Cu") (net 8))
 (segment (start 142.24 96.52) (end 142.748 96.012) (width 0.2) (layer "F.Cu") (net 8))
 (segment (start 139.192 96.52) (end 142.24 96.52) (width 0.2) (layer "F.Cu") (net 8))
 (segment (start 143.256 94.488) (end 162.052 94.488) (width 0.2) (layer "F.Cu") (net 8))
 (segment (start 125.369 69.195) (end 157.881 69.195) (width 0.2) (layer "F.Cu") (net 18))
 (segment (start 163.322 73.411) (end 164.587 74.676) (width 0.2) (layer "F.Cu") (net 18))
 (segment (start 157.881 69.195) (end 158.242 68.834) (width 0.2) (layer "F.Cu") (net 18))
 (segment (start 158.242 68.086) (end 158.496 67.832) (width 0.2) (layer "F.Cu") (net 18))
 (segment (start 124.46 70.104) (end 125.369 69.195) (width 0.2) (layer "F.Cu") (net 18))
 (segment (start 158.496 67.832) (end 162.955 67.832) (width 0.2) (layer "F.Cu") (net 18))
 (segment (start 163.322 68.199) (end 163.322 73.411) (width 0.2) (layer "F.Cu") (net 18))
 (segment (start 158.242 68.834) (end 158.242 68.086) (width 0.2) (layer "F.Cu") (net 18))
 (segment (start 162.955 67.832) (end 163.322 68.199) (width 0.2) (layer "F.Cu") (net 18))
 (segment (start 156.972 72.644) (end 156.972 78.486) (width 0.2) (layer "F.Cu") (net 20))
 (segment (start 156.972 78.486) (end 157.226 78.74) (width 0.2) (layer "F.Cu") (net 20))
 (segment (start 157.226 78.74) (end 158.242 78.74) (width 0.2) (layer "F.Cu") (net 20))
 (segment (start 132.334 79.883) (end 129.032 79.883) (width 0.2) (layer "F.Cu") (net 15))
 (segment (start 127.381 79.375) (end 127.381 77.978) (width 0.2) (layer "F.Cu") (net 15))
 (segment (start 166.116 80.264) (end 132.715 80.264) (width 0.2) (layer "F.Cu") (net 15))
 (segment (start 164.592 69.596) (end 166.624 71.628) (width 0.2) (layer "F.Cu") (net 15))
 (segment (start 129.032 79.883) (end 128.778 79.629) (width 0.2) (layer "F.Cu") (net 15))
 (segment (start 128.778 79.629) (end 127.635 79.629) (width 0.2) (layer "F.Cu") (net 15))
 (segment (start 166.624 79.756) (end 166.116 80.264) (width 0.2) (layer "F.Cu") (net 15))
 (segment (start 166.624 71.628) (end 166.624 79.756) (width 0.2) (layer "F.Cu") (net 15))
 (segment (start 127.127 77.724) (end 124.46 77.724) (width 0.2) (layer "F.Cu") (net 15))
 (segment (start 127.635 79.629) (end 127.381 79.375) (width 0.2) (layer "F.Cu") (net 15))
 (segment (start 127.381 77.978) (end 127.127 77.724) (width 0.2) (layer "F.Cu") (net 15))
 (segment (start 132.715 80.264) (end 132.334 79.883) (width 0.2) (layer "F.Cu") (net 15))
 (segment (start 128.925 80.538) (end 131.592 80.538) (width 0.2) (layer "F.Cu") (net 14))
 (segment (start 124.46 80.264) (end 128.651 80.264) (width 0.2) (layer "F.Cu") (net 14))
 (segment (start 128.651 80.264) (end 128.925 80.538) (width 0.2) (layer "F.Cu") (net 14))
 (via (at 131.592 80.538) (size 0.6) (drill 0.3) (layers "F.Cu" "B.Cu") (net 14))
 (segment (start 167.132 79.883) (end 166.751 80.264) (width 0.2) (layer "B.Cu") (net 14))
 (segment (start 166.751 80.264) (end 166.477 80.538) (width 0.2) (layer "B.Cu") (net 14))
 (segment (start 167.132 69.596) (end 167.132 79.883) (width 0.2) (layer "B.Cu") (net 14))
 (segment (start 166.477 80.538) (end 148.59 80.538) (width 0.2) (layer "B.Cu") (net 14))
 (segment (start 148.59 80.538) (end 131.592 80.538) (width 0.2) (layer "B.Cu") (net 14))
 (segment (start 127.254 73.914) (end 127.254 70.104) (width 0.2) (layer "F.Cu") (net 13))
 (segment (start 127.762 69.596) (end 162.052 69.596) (width 0.2) (layer "F.Cu") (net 13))
 (segment (start 127.254 70.104) (end 127.762 69.596) (width 0.2) (layer "F.Cu") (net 13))
 (via (at 127.254 73.914) (size 0.6) (drill 0.3) (layers "F.Cu" "B.Cu") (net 13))
 (segment (start 126.873 82.804) (end 124.46 82.804) (width 0.2) (layer "B.Cu") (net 13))
 (segment (start 127.254 73.914) (end 127.254 82.423) (width 0.2) (layer "B.Cu") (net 13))
 (segment (start 127.254 82.423) (end 126.873 82.804) (width 0.2) (layer "B.Cu") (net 13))
 (segment (start 131.826 75.184) (end 132.08 75.438) (width 0.2) (layer "F.Cu") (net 16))
 (segment (start 125.295 75.184) (end 131.826 75.184) (width 0.2) (layer "F.Cu") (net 16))
 (segment (start 132.08 75.438) (end 132.08 76.708) (width 0.2) (layer "F.Cu") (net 16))
 (via (at 132.08 76.708) (size 0.6) (drill 0.3) (layers "F.Cu" "B.Cu") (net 16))
 (segment (start 132.08 76.708) (end 132.08 79.756) (width 0.2) (layer "B.Cu") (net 16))
 (segment (start 152.908 80.137) (end 153.162 79.883) (width 0.2) (layer "B.Cu") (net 16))
 (segment (start 132.461 80.137) (end 152.908 80.137) (width 0.2) (layer "B.Cu") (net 16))
 (segment (start 153.162 79.883) (end 153.162 78.74) (width 0.2) (layer "B.Cu") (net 16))
 (segment (start 132.08 79.756) (end 132.461 80.137) (width 0.2) (layer "B.Cu") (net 16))
 (segment (start 146.05 70.612) (end 146.558 71.12) (width 0.2) (layer "F.Cu") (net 2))
 (segment (start 131.318 70.612) (end 130.81 71.12) (width 0.2) (layer "F.Cu") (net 2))
 (segment (start 138.684 71.12) (end 138.176 70.612) (width 0.2) (layer "F.Cu") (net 2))
 (segment (start 153.924 70.612) (end 154.432 71.12) (width 0.2) (layer "F.Cu") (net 2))
 (segment (start 130.81 71.12) (end 130.81 72.644) (width 0.2) (layer "F.Cu") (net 2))
 (segment (start 138.176 70.612) (end 146.05 70.612) (width 0.2) (layer "F.Cu") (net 2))
 (segment (start 138.176 70.612) (end 131.318 70.612) (width 0.2) (layer "F.Cu") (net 2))
 (segment (start 146.558 71.12) (end 146.558 72.644) (width 0.2) (layer "F.Cu") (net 2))
 (segment (start 154.432 71.12) (end 154.432 72.644) (width 0.2) (layer "F.Cu") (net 2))
 (segment (start 146.05 70.612) (end 153.924 70.612) (width 0.2) (layer "F.Cu") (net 2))
 (segment (start 138.684 72.644) (end 138.684 71.12) (width 0.2) (layer "F.Cu") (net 2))
 (segment (start 130.81 72.644) (end 130.81 81.534) (width 0.2) (layer "B.Cu") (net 2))
 (segment (start 131.258 81.982) (end 136.906 81.982) (width 0.2) (layer "B.Cu") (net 2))
 (segment (start 130.81 81.534) (end 131.258 81.982) (width 0.2) (layer "B.Cu") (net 2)))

